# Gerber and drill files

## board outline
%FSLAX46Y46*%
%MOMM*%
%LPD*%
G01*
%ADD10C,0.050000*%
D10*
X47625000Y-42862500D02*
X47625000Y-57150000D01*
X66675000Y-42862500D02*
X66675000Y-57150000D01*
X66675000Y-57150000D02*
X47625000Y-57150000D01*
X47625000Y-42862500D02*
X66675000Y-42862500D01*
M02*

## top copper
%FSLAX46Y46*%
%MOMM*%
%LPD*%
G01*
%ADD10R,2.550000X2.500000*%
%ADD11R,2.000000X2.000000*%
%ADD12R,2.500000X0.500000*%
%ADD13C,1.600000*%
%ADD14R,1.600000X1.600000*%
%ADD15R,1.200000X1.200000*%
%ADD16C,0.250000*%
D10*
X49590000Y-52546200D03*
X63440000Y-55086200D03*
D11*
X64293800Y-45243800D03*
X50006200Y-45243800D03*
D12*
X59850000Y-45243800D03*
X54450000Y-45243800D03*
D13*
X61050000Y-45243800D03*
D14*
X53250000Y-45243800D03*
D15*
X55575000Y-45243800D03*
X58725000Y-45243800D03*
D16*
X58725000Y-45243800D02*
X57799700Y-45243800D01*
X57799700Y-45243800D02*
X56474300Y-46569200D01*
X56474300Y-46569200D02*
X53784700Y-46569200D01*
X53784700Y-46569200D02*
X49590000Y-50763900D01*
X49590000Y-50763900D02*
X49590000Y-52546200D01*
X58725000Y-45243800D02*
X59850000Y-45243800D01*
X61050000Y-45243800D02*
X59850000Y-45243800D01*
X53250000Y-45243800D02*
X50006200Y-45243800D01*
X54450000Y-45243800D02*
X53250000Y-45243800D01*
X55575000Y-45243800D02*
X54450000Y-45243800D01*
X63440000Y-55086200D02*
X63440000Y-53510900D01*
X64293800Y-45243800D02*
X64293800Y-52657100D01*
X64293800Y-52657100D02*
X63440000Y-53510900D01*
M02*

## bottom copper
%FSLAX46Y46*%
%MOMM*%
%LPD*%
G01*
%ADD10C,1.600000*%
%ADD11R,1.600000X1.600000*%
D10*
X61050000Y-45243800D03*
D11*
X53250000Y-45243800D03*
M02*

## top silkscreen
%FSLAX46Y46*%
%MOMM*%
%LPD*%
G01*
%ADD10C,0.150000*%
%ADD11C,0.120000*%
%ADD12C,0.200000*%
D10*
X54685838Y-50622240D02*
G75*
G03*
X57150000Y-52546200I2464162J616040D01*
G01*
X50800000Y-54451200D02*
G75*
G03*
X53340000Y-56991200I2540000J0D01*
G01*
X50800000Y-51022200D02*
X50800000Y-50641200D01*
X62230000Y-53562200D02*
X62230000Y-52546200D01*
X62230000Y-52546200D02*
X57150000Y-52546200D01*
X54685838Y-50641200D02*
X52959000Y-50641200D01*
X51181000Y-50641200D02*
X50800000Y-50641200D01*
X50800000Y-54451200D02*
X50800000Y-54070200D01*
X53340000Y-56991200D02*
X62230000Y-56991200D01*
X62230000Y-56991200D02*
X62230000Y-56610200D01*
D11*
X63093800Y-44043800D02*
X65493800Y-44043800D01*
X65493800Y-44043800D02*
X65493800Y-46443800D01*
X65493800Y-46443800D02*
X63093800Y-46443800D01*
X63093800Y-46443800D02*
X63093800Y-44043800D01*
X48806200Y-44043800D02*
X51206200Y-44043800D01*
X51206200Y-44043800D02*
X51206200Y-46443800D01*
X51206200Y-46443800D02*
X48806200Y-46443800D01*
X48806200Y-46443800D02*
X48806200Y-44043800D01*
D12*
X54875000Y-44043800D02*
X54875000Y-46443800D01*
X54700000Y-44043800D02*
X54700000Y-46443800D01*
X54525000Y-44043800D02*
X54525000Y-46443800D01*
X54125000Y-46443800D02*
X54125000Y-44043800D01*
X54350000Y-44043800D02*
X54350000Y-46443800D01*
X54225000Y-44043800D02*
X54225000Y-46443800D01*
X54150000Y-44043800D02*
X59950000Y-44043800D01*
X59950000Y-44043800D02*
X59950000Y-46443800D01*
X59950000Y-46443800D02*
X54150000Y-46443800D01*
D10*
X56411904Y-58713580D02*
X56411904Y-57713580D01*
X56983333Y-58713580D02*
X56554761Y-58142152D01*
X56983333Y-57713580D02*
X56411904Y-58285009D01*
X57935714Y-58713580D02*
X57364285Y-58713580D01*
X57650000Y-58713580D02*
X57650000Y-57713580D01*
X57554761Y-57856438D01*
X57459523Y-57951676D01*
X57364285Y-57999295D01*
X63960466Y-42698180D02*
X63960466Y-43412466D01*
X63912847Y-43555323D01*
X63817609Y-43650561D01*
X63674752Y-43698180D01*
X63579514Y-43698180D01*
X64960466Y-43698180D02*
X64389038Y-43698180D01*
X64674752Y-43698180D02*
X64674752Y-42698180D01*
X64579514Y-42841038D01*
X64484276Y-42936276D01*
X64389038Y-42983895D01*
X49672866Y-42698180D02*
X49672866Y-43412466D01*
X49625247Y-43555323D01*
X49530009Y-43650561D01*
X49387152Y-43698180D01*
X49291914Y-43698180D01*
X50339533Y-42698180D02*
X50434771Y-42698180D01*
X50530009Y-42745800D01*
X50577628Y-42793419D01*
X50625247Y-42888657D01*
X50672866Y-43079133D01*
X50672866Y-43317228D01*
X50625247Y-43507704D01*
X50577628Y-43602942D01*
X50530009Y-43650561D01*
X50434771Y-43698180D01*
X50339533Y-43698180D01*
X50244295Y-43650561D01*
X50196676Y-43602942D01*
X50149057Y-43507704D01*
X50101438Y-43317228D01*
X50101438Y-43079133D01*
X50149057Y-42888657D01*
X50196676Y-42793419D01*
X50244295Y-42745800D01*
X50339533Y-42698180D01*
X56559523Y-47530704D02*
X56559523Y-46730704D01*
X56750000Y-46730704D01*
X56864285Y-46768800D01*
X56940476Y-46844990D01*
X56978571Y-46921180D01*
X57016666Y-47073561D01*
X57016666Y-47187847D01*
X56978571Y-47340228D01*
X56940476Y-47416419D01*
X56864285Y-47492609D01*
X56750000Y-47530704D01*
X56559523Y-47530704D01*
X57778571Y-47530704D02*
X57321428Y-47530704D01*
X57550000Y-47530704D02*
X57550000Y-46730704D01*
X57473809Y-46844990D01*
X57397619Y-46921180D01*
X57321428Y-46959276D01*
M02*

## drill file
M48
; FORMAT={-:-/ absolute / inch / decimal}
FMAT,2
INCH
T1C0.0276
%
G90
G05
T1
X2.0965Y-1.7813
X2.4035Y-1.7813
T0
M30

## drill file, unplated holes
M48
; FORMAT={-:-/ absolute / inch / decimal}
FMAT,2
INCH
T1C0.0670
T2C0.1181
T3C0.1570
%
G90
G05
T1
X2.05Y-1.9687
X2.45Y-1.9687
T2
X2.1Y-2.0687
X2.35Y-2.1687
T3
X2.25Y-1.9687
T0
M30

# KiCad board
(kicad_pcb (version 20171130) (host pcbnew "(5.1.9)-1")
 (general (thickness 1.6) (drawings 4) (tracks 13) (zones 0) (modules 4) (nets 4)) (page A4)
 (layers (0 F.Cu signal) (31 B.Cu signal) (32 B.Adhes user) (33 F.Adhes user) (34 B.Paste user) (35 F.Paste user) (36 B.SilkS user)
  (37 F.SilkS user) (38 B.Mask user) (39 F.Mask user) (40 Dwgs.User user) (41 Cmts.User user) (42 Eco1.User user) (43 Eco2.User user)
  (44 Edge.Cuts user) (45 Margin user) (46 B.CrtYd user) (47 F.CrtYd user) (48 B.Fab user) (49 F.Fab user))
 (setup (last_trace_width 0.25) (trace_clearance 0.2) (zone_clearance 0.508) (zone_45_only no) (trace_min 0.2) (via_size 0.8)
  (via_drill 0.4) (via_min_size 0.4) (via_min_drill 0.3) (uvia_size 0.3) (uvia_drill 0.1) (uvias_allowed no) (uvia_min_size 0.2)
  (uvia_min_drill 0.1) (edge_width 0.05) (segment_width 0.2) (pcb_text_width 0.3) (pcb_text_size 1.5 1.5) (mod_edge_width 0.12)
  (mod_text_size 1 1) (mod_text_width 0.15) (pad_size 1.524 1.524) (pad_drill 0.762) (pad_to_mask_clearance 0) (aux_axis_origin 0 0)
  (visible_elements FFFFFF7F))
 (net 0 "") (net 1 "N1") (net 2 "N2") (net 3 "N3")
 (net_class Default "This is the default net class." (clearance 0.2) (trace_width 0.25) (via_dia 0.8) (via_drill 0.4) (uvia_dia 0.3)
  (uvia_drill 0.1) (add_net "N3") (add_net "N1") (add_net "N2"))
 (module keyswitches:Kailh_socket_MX (layer B.Cu) (at 57.15 50.0062)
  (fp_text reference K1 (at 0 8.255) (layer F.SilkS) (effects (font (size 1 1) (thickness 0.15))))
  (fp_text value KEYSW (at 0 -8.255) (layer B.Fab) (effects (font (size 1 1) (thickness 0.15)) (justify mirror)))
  (fp_arc (start 0 0) (end 0 2.54) (angle 75.96375653) (layer F.SilkS) (width 0.15))
  (fp_arc (start -3.81 4.445) (end -3.81 6.985) (angle 90) (layer F.SilkS) (width 0.15))
  (fp_line (start -6.35 1.016) (end -6.35 0.635) (layer F.SilkS) (width 0.15))
  (fp_line (start 5.08 3.556) (end 5.08 2.54) (layer F.SilkS) (width 0.15))
  (fp_line (start 5.08 2.54) (end 0 2.54) (layer F.SilkS) (width 0.15))
  (fp_line (start -2.464162 0.635) (end -4.191 0.635) (layer F.SilkS) (width 0.15))
  (fp_line (start -5.969 0.635) (end -6.35 0.635) (layer F.SilkS) (width 0.15))
  (fp_line (start -6.35 4.445) (end -6.35 4.064) (layer F.SilkS) (width 0.15))
  (fp_line (start -3.81 6.985) (end 5.08 6.985) (layer F.SilkS) (width 0.15))
  (fp_line (start 5.08 6.985) (end 5.08 6.604) (layer F.SilkS) (width 0.15))
  (pad 2 smd rect (at -7.56 2.54) (size 2.55 2.5) (layers F.Cu F.Paste F.Mask) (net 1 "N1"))
  (pad "" np_thru_hole circle (at -5.08 0) (size 1.7018 1.7018) (drill 1.7018) (layers *.Cu *.Mask))
  (pad "" np_thru_hole circle (at 5.08 0) (size 1.7018 1.7018) (drill 1.7018) (layers *.Cu *.Mask))
  (pad "" np_thru_hole circle (at 0 0) (size 3.9878 3.9878) (drill 3.9878) (layers *.Cu *.Mask))
  (pad "" np_thru_hole circle (at -3.81 2.54) (size 3 3) (drill 3) (layers *.Cu *.Mask))
  (pad "" np_thru_hole circle (at 2.54 5.08) (size 3 3) (drill 3) (layers *.Cu *.Mask))
  (pad 1 smd rect (at 6.29 5.08) (size 2.55 2.5) (layers F.Cu F.Paste F.Mask) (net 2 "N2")))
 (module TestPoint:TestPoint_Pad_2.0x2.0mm (layer F.Cu) (at 64.2938 45.2438)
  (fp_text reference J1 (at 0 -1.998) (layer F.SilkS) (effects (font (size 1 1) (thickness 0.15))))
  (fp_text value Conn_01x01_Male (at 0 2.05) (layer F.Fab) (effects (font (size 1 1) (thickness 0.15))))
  (fp_line (start -1.2 -1.2) (end 1.2 -1.2) (layer F.SilkS) (width 0.12))
  (fp_line (start 1.2 -1.2) (end 1.2 1.2) (layer F.SilkS) (width 0.12))
  (fp_line (start 1.2 1.2) (end -1.2 1.2) (layer F.SilkS) (width 0.12))
  (fp_line (start -1.2 1.2) (end -1.2 -1.2) (layer F.SilkS) (width 0.12))
  (pad 1 smd rect (at 0 0) (size 2 2) (layers F.Cu F.Mask) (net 2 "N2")))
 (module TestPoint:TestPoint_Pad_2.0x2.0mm (layer F.Cu) (at 50.0062 45.2438)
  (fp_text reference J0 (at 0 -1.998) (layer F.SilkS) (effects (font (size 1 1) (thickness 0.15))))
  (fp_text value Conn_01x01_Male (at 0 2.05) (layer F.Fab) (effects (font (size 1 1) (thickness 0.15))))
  (fp_line (start -1.2 -1.2) (end 1.2 -1.2) (layer F.SilkS) (width 0.12))
  (fp_line (start 1.2 -1.2) (end 1.2 1.2) (layer F.SilkS) (width 0.12))
  (fp_line (start 1.2 1.2) (end -1.2 1.2) (layer F.SilkS) (width 0.12))
  (fp_line (start -1.2 1.2) (end -1.2 -1.2) (layer F.SilkS) (width 0.12))
  (pad 1 smd rect (at 0 0) (size 2 2) (layers F.Cu F.Mask) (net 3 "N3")))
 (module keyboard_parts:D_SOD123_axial (layer F.Cu) (at 57.15 45.2438)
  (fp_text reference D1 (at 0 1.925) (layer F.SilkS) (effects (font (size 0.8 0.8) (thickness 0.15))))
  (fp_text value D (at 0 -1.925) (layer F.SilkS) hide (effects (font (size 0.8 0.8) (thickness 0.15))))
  (fp_line (start -2.275 -1.2) (end -2.275 1.2) (layer F.SilkS) (width 0.2))
  (fp_line (start -2.45 -1.2) (end -2.45 1.2) (layer F.SilkS) (width 0.2))
  (fp_line (start -2.625 -1.2) (end -2.625 1.2) (layer F.SilkS) (width 0.2))
  (fp_line (start -3.025 1.2) (end -3.025 -1.2) (layer F.SilkS) (width 0.2))
  (fp_line (start -2.8 -1.2) (end -2.8 1.2) (layer F.SilkS) (width 0.2))
  (fp_line (start -2.925 -1.2) (end -2.925 1.2) (layer F.SilkS) (width 0.2))
  (fp_line (start -3 -1.2) (end 2.8 -1.2) (layer F.SilkS) (width 0.2))
  (fp_line (start 2.8 -1.2) (end 2.8 1.2) (layer F.SilkS) (width 0.2))
  (fp_line (start 2.8 1.2) (end -3 1.2) (layer F.SilkS) (width 0.2))
  (pad 2 smd rect (at 2.7 0) (size 2.5 0.5) (layers F.Cu) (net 1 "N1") (solder_mask_margin -999))
  (pad 1 smd rect (at -2.7 0) (size 2.5 0.5) (layers F.Cu) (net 3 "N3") (solder_mask_margin -999))
  (pad 2 thru_hole circle (at 3.9 0) (size 1.6 1.6) (drill 0.7) (layers *.Cu *.Mask F.SilkS) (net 1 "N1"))
  (pad 1 thru_hole rect (at -3.9 0) (size 1.6 1.6) (drill 0.7) (layers *.Cu *.Mask F.SilkS) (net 3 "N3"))
  (pad 1 smd rect (at -1.575 0) (size 1.2 1.2) (layers F.Cu F.Paste F.Mask) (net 3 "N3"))
  (pad 2 smd rect (at 1.575 0) (size 1.2 1.2) (layers F.Cu F.Paste F.Mask) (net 1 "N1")))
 (gr_line (start 47.625 42.8625) (end 47.625 57.15) (layer Edge.Cuts) (width 0.05))
 (gr_line (start 66.675 42.8625) (end 66.675 57.15) (layer Edge.Cuts) (width 0.05))
 (gr_line (start 66.675 57.15) (end 47.625 57.15) (layer Edge.Cuts) (width 0.05))
 (gr_line (start 47.625 42.8625) (end 66.675 42.8625) (layer Edge.Cuts) (width 0.05))
 (segment (start 58.725 45.2438) (end 57.7997 45.2438) (width 0.25) (layer F.Cu) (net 1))
 (segment (start 57.7997 45.2438) (end 56.4743 46.5692) (width 0.25) (layer F.Cu) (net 1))
 (segment (start 56.4743 46.5692) (end 53.7847 46.5692) (width 0.25) (layer F.Cu) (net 1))
 (segment (start 53.7847 46.5692) (end 49.59 50.7639) (width 0.25) (layer F.Cu) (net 1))
 (segment (start 49.59 50.7639) (end 49.59 52.5462) (width 0.25) (layer F.Cu) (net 1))
 (segment (start 58.725 45.2438) (end 59.85 45.2438) (width 0.25) (layer F.Cu) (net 1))
 (segment (start 61.05 45.2438) (end 59.85 45.2438) (width 0.25) (layer F.Cu) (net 1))
 (segment (start 53.25 45.2438) (end 50.0062 45.2438) (width 0.25) (layer F.Cu) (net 3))
 (segment (start 54.45 45.2438) (end 53.25 45.2438) (width 0.25) (layer F.Cu) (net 3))
 (segment (start 55.575 45.2438) (end 54.45 45.2438) (width 0.25) (layer F.Cu) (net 3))
 (segment (start 63.44 55.0862) (end 63.44 53.5109) (width 0.25) (layer F.Cu) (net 2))
 (segment (start 64.2938 45.2438) (end 64.2938 52.6571) (width 0.25) (layer F.Cu) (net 2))
 (segment (start 64.2938 52.6571) (end 63.44 53.5109) (width 0.25) (layer F.Cu) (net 2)))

